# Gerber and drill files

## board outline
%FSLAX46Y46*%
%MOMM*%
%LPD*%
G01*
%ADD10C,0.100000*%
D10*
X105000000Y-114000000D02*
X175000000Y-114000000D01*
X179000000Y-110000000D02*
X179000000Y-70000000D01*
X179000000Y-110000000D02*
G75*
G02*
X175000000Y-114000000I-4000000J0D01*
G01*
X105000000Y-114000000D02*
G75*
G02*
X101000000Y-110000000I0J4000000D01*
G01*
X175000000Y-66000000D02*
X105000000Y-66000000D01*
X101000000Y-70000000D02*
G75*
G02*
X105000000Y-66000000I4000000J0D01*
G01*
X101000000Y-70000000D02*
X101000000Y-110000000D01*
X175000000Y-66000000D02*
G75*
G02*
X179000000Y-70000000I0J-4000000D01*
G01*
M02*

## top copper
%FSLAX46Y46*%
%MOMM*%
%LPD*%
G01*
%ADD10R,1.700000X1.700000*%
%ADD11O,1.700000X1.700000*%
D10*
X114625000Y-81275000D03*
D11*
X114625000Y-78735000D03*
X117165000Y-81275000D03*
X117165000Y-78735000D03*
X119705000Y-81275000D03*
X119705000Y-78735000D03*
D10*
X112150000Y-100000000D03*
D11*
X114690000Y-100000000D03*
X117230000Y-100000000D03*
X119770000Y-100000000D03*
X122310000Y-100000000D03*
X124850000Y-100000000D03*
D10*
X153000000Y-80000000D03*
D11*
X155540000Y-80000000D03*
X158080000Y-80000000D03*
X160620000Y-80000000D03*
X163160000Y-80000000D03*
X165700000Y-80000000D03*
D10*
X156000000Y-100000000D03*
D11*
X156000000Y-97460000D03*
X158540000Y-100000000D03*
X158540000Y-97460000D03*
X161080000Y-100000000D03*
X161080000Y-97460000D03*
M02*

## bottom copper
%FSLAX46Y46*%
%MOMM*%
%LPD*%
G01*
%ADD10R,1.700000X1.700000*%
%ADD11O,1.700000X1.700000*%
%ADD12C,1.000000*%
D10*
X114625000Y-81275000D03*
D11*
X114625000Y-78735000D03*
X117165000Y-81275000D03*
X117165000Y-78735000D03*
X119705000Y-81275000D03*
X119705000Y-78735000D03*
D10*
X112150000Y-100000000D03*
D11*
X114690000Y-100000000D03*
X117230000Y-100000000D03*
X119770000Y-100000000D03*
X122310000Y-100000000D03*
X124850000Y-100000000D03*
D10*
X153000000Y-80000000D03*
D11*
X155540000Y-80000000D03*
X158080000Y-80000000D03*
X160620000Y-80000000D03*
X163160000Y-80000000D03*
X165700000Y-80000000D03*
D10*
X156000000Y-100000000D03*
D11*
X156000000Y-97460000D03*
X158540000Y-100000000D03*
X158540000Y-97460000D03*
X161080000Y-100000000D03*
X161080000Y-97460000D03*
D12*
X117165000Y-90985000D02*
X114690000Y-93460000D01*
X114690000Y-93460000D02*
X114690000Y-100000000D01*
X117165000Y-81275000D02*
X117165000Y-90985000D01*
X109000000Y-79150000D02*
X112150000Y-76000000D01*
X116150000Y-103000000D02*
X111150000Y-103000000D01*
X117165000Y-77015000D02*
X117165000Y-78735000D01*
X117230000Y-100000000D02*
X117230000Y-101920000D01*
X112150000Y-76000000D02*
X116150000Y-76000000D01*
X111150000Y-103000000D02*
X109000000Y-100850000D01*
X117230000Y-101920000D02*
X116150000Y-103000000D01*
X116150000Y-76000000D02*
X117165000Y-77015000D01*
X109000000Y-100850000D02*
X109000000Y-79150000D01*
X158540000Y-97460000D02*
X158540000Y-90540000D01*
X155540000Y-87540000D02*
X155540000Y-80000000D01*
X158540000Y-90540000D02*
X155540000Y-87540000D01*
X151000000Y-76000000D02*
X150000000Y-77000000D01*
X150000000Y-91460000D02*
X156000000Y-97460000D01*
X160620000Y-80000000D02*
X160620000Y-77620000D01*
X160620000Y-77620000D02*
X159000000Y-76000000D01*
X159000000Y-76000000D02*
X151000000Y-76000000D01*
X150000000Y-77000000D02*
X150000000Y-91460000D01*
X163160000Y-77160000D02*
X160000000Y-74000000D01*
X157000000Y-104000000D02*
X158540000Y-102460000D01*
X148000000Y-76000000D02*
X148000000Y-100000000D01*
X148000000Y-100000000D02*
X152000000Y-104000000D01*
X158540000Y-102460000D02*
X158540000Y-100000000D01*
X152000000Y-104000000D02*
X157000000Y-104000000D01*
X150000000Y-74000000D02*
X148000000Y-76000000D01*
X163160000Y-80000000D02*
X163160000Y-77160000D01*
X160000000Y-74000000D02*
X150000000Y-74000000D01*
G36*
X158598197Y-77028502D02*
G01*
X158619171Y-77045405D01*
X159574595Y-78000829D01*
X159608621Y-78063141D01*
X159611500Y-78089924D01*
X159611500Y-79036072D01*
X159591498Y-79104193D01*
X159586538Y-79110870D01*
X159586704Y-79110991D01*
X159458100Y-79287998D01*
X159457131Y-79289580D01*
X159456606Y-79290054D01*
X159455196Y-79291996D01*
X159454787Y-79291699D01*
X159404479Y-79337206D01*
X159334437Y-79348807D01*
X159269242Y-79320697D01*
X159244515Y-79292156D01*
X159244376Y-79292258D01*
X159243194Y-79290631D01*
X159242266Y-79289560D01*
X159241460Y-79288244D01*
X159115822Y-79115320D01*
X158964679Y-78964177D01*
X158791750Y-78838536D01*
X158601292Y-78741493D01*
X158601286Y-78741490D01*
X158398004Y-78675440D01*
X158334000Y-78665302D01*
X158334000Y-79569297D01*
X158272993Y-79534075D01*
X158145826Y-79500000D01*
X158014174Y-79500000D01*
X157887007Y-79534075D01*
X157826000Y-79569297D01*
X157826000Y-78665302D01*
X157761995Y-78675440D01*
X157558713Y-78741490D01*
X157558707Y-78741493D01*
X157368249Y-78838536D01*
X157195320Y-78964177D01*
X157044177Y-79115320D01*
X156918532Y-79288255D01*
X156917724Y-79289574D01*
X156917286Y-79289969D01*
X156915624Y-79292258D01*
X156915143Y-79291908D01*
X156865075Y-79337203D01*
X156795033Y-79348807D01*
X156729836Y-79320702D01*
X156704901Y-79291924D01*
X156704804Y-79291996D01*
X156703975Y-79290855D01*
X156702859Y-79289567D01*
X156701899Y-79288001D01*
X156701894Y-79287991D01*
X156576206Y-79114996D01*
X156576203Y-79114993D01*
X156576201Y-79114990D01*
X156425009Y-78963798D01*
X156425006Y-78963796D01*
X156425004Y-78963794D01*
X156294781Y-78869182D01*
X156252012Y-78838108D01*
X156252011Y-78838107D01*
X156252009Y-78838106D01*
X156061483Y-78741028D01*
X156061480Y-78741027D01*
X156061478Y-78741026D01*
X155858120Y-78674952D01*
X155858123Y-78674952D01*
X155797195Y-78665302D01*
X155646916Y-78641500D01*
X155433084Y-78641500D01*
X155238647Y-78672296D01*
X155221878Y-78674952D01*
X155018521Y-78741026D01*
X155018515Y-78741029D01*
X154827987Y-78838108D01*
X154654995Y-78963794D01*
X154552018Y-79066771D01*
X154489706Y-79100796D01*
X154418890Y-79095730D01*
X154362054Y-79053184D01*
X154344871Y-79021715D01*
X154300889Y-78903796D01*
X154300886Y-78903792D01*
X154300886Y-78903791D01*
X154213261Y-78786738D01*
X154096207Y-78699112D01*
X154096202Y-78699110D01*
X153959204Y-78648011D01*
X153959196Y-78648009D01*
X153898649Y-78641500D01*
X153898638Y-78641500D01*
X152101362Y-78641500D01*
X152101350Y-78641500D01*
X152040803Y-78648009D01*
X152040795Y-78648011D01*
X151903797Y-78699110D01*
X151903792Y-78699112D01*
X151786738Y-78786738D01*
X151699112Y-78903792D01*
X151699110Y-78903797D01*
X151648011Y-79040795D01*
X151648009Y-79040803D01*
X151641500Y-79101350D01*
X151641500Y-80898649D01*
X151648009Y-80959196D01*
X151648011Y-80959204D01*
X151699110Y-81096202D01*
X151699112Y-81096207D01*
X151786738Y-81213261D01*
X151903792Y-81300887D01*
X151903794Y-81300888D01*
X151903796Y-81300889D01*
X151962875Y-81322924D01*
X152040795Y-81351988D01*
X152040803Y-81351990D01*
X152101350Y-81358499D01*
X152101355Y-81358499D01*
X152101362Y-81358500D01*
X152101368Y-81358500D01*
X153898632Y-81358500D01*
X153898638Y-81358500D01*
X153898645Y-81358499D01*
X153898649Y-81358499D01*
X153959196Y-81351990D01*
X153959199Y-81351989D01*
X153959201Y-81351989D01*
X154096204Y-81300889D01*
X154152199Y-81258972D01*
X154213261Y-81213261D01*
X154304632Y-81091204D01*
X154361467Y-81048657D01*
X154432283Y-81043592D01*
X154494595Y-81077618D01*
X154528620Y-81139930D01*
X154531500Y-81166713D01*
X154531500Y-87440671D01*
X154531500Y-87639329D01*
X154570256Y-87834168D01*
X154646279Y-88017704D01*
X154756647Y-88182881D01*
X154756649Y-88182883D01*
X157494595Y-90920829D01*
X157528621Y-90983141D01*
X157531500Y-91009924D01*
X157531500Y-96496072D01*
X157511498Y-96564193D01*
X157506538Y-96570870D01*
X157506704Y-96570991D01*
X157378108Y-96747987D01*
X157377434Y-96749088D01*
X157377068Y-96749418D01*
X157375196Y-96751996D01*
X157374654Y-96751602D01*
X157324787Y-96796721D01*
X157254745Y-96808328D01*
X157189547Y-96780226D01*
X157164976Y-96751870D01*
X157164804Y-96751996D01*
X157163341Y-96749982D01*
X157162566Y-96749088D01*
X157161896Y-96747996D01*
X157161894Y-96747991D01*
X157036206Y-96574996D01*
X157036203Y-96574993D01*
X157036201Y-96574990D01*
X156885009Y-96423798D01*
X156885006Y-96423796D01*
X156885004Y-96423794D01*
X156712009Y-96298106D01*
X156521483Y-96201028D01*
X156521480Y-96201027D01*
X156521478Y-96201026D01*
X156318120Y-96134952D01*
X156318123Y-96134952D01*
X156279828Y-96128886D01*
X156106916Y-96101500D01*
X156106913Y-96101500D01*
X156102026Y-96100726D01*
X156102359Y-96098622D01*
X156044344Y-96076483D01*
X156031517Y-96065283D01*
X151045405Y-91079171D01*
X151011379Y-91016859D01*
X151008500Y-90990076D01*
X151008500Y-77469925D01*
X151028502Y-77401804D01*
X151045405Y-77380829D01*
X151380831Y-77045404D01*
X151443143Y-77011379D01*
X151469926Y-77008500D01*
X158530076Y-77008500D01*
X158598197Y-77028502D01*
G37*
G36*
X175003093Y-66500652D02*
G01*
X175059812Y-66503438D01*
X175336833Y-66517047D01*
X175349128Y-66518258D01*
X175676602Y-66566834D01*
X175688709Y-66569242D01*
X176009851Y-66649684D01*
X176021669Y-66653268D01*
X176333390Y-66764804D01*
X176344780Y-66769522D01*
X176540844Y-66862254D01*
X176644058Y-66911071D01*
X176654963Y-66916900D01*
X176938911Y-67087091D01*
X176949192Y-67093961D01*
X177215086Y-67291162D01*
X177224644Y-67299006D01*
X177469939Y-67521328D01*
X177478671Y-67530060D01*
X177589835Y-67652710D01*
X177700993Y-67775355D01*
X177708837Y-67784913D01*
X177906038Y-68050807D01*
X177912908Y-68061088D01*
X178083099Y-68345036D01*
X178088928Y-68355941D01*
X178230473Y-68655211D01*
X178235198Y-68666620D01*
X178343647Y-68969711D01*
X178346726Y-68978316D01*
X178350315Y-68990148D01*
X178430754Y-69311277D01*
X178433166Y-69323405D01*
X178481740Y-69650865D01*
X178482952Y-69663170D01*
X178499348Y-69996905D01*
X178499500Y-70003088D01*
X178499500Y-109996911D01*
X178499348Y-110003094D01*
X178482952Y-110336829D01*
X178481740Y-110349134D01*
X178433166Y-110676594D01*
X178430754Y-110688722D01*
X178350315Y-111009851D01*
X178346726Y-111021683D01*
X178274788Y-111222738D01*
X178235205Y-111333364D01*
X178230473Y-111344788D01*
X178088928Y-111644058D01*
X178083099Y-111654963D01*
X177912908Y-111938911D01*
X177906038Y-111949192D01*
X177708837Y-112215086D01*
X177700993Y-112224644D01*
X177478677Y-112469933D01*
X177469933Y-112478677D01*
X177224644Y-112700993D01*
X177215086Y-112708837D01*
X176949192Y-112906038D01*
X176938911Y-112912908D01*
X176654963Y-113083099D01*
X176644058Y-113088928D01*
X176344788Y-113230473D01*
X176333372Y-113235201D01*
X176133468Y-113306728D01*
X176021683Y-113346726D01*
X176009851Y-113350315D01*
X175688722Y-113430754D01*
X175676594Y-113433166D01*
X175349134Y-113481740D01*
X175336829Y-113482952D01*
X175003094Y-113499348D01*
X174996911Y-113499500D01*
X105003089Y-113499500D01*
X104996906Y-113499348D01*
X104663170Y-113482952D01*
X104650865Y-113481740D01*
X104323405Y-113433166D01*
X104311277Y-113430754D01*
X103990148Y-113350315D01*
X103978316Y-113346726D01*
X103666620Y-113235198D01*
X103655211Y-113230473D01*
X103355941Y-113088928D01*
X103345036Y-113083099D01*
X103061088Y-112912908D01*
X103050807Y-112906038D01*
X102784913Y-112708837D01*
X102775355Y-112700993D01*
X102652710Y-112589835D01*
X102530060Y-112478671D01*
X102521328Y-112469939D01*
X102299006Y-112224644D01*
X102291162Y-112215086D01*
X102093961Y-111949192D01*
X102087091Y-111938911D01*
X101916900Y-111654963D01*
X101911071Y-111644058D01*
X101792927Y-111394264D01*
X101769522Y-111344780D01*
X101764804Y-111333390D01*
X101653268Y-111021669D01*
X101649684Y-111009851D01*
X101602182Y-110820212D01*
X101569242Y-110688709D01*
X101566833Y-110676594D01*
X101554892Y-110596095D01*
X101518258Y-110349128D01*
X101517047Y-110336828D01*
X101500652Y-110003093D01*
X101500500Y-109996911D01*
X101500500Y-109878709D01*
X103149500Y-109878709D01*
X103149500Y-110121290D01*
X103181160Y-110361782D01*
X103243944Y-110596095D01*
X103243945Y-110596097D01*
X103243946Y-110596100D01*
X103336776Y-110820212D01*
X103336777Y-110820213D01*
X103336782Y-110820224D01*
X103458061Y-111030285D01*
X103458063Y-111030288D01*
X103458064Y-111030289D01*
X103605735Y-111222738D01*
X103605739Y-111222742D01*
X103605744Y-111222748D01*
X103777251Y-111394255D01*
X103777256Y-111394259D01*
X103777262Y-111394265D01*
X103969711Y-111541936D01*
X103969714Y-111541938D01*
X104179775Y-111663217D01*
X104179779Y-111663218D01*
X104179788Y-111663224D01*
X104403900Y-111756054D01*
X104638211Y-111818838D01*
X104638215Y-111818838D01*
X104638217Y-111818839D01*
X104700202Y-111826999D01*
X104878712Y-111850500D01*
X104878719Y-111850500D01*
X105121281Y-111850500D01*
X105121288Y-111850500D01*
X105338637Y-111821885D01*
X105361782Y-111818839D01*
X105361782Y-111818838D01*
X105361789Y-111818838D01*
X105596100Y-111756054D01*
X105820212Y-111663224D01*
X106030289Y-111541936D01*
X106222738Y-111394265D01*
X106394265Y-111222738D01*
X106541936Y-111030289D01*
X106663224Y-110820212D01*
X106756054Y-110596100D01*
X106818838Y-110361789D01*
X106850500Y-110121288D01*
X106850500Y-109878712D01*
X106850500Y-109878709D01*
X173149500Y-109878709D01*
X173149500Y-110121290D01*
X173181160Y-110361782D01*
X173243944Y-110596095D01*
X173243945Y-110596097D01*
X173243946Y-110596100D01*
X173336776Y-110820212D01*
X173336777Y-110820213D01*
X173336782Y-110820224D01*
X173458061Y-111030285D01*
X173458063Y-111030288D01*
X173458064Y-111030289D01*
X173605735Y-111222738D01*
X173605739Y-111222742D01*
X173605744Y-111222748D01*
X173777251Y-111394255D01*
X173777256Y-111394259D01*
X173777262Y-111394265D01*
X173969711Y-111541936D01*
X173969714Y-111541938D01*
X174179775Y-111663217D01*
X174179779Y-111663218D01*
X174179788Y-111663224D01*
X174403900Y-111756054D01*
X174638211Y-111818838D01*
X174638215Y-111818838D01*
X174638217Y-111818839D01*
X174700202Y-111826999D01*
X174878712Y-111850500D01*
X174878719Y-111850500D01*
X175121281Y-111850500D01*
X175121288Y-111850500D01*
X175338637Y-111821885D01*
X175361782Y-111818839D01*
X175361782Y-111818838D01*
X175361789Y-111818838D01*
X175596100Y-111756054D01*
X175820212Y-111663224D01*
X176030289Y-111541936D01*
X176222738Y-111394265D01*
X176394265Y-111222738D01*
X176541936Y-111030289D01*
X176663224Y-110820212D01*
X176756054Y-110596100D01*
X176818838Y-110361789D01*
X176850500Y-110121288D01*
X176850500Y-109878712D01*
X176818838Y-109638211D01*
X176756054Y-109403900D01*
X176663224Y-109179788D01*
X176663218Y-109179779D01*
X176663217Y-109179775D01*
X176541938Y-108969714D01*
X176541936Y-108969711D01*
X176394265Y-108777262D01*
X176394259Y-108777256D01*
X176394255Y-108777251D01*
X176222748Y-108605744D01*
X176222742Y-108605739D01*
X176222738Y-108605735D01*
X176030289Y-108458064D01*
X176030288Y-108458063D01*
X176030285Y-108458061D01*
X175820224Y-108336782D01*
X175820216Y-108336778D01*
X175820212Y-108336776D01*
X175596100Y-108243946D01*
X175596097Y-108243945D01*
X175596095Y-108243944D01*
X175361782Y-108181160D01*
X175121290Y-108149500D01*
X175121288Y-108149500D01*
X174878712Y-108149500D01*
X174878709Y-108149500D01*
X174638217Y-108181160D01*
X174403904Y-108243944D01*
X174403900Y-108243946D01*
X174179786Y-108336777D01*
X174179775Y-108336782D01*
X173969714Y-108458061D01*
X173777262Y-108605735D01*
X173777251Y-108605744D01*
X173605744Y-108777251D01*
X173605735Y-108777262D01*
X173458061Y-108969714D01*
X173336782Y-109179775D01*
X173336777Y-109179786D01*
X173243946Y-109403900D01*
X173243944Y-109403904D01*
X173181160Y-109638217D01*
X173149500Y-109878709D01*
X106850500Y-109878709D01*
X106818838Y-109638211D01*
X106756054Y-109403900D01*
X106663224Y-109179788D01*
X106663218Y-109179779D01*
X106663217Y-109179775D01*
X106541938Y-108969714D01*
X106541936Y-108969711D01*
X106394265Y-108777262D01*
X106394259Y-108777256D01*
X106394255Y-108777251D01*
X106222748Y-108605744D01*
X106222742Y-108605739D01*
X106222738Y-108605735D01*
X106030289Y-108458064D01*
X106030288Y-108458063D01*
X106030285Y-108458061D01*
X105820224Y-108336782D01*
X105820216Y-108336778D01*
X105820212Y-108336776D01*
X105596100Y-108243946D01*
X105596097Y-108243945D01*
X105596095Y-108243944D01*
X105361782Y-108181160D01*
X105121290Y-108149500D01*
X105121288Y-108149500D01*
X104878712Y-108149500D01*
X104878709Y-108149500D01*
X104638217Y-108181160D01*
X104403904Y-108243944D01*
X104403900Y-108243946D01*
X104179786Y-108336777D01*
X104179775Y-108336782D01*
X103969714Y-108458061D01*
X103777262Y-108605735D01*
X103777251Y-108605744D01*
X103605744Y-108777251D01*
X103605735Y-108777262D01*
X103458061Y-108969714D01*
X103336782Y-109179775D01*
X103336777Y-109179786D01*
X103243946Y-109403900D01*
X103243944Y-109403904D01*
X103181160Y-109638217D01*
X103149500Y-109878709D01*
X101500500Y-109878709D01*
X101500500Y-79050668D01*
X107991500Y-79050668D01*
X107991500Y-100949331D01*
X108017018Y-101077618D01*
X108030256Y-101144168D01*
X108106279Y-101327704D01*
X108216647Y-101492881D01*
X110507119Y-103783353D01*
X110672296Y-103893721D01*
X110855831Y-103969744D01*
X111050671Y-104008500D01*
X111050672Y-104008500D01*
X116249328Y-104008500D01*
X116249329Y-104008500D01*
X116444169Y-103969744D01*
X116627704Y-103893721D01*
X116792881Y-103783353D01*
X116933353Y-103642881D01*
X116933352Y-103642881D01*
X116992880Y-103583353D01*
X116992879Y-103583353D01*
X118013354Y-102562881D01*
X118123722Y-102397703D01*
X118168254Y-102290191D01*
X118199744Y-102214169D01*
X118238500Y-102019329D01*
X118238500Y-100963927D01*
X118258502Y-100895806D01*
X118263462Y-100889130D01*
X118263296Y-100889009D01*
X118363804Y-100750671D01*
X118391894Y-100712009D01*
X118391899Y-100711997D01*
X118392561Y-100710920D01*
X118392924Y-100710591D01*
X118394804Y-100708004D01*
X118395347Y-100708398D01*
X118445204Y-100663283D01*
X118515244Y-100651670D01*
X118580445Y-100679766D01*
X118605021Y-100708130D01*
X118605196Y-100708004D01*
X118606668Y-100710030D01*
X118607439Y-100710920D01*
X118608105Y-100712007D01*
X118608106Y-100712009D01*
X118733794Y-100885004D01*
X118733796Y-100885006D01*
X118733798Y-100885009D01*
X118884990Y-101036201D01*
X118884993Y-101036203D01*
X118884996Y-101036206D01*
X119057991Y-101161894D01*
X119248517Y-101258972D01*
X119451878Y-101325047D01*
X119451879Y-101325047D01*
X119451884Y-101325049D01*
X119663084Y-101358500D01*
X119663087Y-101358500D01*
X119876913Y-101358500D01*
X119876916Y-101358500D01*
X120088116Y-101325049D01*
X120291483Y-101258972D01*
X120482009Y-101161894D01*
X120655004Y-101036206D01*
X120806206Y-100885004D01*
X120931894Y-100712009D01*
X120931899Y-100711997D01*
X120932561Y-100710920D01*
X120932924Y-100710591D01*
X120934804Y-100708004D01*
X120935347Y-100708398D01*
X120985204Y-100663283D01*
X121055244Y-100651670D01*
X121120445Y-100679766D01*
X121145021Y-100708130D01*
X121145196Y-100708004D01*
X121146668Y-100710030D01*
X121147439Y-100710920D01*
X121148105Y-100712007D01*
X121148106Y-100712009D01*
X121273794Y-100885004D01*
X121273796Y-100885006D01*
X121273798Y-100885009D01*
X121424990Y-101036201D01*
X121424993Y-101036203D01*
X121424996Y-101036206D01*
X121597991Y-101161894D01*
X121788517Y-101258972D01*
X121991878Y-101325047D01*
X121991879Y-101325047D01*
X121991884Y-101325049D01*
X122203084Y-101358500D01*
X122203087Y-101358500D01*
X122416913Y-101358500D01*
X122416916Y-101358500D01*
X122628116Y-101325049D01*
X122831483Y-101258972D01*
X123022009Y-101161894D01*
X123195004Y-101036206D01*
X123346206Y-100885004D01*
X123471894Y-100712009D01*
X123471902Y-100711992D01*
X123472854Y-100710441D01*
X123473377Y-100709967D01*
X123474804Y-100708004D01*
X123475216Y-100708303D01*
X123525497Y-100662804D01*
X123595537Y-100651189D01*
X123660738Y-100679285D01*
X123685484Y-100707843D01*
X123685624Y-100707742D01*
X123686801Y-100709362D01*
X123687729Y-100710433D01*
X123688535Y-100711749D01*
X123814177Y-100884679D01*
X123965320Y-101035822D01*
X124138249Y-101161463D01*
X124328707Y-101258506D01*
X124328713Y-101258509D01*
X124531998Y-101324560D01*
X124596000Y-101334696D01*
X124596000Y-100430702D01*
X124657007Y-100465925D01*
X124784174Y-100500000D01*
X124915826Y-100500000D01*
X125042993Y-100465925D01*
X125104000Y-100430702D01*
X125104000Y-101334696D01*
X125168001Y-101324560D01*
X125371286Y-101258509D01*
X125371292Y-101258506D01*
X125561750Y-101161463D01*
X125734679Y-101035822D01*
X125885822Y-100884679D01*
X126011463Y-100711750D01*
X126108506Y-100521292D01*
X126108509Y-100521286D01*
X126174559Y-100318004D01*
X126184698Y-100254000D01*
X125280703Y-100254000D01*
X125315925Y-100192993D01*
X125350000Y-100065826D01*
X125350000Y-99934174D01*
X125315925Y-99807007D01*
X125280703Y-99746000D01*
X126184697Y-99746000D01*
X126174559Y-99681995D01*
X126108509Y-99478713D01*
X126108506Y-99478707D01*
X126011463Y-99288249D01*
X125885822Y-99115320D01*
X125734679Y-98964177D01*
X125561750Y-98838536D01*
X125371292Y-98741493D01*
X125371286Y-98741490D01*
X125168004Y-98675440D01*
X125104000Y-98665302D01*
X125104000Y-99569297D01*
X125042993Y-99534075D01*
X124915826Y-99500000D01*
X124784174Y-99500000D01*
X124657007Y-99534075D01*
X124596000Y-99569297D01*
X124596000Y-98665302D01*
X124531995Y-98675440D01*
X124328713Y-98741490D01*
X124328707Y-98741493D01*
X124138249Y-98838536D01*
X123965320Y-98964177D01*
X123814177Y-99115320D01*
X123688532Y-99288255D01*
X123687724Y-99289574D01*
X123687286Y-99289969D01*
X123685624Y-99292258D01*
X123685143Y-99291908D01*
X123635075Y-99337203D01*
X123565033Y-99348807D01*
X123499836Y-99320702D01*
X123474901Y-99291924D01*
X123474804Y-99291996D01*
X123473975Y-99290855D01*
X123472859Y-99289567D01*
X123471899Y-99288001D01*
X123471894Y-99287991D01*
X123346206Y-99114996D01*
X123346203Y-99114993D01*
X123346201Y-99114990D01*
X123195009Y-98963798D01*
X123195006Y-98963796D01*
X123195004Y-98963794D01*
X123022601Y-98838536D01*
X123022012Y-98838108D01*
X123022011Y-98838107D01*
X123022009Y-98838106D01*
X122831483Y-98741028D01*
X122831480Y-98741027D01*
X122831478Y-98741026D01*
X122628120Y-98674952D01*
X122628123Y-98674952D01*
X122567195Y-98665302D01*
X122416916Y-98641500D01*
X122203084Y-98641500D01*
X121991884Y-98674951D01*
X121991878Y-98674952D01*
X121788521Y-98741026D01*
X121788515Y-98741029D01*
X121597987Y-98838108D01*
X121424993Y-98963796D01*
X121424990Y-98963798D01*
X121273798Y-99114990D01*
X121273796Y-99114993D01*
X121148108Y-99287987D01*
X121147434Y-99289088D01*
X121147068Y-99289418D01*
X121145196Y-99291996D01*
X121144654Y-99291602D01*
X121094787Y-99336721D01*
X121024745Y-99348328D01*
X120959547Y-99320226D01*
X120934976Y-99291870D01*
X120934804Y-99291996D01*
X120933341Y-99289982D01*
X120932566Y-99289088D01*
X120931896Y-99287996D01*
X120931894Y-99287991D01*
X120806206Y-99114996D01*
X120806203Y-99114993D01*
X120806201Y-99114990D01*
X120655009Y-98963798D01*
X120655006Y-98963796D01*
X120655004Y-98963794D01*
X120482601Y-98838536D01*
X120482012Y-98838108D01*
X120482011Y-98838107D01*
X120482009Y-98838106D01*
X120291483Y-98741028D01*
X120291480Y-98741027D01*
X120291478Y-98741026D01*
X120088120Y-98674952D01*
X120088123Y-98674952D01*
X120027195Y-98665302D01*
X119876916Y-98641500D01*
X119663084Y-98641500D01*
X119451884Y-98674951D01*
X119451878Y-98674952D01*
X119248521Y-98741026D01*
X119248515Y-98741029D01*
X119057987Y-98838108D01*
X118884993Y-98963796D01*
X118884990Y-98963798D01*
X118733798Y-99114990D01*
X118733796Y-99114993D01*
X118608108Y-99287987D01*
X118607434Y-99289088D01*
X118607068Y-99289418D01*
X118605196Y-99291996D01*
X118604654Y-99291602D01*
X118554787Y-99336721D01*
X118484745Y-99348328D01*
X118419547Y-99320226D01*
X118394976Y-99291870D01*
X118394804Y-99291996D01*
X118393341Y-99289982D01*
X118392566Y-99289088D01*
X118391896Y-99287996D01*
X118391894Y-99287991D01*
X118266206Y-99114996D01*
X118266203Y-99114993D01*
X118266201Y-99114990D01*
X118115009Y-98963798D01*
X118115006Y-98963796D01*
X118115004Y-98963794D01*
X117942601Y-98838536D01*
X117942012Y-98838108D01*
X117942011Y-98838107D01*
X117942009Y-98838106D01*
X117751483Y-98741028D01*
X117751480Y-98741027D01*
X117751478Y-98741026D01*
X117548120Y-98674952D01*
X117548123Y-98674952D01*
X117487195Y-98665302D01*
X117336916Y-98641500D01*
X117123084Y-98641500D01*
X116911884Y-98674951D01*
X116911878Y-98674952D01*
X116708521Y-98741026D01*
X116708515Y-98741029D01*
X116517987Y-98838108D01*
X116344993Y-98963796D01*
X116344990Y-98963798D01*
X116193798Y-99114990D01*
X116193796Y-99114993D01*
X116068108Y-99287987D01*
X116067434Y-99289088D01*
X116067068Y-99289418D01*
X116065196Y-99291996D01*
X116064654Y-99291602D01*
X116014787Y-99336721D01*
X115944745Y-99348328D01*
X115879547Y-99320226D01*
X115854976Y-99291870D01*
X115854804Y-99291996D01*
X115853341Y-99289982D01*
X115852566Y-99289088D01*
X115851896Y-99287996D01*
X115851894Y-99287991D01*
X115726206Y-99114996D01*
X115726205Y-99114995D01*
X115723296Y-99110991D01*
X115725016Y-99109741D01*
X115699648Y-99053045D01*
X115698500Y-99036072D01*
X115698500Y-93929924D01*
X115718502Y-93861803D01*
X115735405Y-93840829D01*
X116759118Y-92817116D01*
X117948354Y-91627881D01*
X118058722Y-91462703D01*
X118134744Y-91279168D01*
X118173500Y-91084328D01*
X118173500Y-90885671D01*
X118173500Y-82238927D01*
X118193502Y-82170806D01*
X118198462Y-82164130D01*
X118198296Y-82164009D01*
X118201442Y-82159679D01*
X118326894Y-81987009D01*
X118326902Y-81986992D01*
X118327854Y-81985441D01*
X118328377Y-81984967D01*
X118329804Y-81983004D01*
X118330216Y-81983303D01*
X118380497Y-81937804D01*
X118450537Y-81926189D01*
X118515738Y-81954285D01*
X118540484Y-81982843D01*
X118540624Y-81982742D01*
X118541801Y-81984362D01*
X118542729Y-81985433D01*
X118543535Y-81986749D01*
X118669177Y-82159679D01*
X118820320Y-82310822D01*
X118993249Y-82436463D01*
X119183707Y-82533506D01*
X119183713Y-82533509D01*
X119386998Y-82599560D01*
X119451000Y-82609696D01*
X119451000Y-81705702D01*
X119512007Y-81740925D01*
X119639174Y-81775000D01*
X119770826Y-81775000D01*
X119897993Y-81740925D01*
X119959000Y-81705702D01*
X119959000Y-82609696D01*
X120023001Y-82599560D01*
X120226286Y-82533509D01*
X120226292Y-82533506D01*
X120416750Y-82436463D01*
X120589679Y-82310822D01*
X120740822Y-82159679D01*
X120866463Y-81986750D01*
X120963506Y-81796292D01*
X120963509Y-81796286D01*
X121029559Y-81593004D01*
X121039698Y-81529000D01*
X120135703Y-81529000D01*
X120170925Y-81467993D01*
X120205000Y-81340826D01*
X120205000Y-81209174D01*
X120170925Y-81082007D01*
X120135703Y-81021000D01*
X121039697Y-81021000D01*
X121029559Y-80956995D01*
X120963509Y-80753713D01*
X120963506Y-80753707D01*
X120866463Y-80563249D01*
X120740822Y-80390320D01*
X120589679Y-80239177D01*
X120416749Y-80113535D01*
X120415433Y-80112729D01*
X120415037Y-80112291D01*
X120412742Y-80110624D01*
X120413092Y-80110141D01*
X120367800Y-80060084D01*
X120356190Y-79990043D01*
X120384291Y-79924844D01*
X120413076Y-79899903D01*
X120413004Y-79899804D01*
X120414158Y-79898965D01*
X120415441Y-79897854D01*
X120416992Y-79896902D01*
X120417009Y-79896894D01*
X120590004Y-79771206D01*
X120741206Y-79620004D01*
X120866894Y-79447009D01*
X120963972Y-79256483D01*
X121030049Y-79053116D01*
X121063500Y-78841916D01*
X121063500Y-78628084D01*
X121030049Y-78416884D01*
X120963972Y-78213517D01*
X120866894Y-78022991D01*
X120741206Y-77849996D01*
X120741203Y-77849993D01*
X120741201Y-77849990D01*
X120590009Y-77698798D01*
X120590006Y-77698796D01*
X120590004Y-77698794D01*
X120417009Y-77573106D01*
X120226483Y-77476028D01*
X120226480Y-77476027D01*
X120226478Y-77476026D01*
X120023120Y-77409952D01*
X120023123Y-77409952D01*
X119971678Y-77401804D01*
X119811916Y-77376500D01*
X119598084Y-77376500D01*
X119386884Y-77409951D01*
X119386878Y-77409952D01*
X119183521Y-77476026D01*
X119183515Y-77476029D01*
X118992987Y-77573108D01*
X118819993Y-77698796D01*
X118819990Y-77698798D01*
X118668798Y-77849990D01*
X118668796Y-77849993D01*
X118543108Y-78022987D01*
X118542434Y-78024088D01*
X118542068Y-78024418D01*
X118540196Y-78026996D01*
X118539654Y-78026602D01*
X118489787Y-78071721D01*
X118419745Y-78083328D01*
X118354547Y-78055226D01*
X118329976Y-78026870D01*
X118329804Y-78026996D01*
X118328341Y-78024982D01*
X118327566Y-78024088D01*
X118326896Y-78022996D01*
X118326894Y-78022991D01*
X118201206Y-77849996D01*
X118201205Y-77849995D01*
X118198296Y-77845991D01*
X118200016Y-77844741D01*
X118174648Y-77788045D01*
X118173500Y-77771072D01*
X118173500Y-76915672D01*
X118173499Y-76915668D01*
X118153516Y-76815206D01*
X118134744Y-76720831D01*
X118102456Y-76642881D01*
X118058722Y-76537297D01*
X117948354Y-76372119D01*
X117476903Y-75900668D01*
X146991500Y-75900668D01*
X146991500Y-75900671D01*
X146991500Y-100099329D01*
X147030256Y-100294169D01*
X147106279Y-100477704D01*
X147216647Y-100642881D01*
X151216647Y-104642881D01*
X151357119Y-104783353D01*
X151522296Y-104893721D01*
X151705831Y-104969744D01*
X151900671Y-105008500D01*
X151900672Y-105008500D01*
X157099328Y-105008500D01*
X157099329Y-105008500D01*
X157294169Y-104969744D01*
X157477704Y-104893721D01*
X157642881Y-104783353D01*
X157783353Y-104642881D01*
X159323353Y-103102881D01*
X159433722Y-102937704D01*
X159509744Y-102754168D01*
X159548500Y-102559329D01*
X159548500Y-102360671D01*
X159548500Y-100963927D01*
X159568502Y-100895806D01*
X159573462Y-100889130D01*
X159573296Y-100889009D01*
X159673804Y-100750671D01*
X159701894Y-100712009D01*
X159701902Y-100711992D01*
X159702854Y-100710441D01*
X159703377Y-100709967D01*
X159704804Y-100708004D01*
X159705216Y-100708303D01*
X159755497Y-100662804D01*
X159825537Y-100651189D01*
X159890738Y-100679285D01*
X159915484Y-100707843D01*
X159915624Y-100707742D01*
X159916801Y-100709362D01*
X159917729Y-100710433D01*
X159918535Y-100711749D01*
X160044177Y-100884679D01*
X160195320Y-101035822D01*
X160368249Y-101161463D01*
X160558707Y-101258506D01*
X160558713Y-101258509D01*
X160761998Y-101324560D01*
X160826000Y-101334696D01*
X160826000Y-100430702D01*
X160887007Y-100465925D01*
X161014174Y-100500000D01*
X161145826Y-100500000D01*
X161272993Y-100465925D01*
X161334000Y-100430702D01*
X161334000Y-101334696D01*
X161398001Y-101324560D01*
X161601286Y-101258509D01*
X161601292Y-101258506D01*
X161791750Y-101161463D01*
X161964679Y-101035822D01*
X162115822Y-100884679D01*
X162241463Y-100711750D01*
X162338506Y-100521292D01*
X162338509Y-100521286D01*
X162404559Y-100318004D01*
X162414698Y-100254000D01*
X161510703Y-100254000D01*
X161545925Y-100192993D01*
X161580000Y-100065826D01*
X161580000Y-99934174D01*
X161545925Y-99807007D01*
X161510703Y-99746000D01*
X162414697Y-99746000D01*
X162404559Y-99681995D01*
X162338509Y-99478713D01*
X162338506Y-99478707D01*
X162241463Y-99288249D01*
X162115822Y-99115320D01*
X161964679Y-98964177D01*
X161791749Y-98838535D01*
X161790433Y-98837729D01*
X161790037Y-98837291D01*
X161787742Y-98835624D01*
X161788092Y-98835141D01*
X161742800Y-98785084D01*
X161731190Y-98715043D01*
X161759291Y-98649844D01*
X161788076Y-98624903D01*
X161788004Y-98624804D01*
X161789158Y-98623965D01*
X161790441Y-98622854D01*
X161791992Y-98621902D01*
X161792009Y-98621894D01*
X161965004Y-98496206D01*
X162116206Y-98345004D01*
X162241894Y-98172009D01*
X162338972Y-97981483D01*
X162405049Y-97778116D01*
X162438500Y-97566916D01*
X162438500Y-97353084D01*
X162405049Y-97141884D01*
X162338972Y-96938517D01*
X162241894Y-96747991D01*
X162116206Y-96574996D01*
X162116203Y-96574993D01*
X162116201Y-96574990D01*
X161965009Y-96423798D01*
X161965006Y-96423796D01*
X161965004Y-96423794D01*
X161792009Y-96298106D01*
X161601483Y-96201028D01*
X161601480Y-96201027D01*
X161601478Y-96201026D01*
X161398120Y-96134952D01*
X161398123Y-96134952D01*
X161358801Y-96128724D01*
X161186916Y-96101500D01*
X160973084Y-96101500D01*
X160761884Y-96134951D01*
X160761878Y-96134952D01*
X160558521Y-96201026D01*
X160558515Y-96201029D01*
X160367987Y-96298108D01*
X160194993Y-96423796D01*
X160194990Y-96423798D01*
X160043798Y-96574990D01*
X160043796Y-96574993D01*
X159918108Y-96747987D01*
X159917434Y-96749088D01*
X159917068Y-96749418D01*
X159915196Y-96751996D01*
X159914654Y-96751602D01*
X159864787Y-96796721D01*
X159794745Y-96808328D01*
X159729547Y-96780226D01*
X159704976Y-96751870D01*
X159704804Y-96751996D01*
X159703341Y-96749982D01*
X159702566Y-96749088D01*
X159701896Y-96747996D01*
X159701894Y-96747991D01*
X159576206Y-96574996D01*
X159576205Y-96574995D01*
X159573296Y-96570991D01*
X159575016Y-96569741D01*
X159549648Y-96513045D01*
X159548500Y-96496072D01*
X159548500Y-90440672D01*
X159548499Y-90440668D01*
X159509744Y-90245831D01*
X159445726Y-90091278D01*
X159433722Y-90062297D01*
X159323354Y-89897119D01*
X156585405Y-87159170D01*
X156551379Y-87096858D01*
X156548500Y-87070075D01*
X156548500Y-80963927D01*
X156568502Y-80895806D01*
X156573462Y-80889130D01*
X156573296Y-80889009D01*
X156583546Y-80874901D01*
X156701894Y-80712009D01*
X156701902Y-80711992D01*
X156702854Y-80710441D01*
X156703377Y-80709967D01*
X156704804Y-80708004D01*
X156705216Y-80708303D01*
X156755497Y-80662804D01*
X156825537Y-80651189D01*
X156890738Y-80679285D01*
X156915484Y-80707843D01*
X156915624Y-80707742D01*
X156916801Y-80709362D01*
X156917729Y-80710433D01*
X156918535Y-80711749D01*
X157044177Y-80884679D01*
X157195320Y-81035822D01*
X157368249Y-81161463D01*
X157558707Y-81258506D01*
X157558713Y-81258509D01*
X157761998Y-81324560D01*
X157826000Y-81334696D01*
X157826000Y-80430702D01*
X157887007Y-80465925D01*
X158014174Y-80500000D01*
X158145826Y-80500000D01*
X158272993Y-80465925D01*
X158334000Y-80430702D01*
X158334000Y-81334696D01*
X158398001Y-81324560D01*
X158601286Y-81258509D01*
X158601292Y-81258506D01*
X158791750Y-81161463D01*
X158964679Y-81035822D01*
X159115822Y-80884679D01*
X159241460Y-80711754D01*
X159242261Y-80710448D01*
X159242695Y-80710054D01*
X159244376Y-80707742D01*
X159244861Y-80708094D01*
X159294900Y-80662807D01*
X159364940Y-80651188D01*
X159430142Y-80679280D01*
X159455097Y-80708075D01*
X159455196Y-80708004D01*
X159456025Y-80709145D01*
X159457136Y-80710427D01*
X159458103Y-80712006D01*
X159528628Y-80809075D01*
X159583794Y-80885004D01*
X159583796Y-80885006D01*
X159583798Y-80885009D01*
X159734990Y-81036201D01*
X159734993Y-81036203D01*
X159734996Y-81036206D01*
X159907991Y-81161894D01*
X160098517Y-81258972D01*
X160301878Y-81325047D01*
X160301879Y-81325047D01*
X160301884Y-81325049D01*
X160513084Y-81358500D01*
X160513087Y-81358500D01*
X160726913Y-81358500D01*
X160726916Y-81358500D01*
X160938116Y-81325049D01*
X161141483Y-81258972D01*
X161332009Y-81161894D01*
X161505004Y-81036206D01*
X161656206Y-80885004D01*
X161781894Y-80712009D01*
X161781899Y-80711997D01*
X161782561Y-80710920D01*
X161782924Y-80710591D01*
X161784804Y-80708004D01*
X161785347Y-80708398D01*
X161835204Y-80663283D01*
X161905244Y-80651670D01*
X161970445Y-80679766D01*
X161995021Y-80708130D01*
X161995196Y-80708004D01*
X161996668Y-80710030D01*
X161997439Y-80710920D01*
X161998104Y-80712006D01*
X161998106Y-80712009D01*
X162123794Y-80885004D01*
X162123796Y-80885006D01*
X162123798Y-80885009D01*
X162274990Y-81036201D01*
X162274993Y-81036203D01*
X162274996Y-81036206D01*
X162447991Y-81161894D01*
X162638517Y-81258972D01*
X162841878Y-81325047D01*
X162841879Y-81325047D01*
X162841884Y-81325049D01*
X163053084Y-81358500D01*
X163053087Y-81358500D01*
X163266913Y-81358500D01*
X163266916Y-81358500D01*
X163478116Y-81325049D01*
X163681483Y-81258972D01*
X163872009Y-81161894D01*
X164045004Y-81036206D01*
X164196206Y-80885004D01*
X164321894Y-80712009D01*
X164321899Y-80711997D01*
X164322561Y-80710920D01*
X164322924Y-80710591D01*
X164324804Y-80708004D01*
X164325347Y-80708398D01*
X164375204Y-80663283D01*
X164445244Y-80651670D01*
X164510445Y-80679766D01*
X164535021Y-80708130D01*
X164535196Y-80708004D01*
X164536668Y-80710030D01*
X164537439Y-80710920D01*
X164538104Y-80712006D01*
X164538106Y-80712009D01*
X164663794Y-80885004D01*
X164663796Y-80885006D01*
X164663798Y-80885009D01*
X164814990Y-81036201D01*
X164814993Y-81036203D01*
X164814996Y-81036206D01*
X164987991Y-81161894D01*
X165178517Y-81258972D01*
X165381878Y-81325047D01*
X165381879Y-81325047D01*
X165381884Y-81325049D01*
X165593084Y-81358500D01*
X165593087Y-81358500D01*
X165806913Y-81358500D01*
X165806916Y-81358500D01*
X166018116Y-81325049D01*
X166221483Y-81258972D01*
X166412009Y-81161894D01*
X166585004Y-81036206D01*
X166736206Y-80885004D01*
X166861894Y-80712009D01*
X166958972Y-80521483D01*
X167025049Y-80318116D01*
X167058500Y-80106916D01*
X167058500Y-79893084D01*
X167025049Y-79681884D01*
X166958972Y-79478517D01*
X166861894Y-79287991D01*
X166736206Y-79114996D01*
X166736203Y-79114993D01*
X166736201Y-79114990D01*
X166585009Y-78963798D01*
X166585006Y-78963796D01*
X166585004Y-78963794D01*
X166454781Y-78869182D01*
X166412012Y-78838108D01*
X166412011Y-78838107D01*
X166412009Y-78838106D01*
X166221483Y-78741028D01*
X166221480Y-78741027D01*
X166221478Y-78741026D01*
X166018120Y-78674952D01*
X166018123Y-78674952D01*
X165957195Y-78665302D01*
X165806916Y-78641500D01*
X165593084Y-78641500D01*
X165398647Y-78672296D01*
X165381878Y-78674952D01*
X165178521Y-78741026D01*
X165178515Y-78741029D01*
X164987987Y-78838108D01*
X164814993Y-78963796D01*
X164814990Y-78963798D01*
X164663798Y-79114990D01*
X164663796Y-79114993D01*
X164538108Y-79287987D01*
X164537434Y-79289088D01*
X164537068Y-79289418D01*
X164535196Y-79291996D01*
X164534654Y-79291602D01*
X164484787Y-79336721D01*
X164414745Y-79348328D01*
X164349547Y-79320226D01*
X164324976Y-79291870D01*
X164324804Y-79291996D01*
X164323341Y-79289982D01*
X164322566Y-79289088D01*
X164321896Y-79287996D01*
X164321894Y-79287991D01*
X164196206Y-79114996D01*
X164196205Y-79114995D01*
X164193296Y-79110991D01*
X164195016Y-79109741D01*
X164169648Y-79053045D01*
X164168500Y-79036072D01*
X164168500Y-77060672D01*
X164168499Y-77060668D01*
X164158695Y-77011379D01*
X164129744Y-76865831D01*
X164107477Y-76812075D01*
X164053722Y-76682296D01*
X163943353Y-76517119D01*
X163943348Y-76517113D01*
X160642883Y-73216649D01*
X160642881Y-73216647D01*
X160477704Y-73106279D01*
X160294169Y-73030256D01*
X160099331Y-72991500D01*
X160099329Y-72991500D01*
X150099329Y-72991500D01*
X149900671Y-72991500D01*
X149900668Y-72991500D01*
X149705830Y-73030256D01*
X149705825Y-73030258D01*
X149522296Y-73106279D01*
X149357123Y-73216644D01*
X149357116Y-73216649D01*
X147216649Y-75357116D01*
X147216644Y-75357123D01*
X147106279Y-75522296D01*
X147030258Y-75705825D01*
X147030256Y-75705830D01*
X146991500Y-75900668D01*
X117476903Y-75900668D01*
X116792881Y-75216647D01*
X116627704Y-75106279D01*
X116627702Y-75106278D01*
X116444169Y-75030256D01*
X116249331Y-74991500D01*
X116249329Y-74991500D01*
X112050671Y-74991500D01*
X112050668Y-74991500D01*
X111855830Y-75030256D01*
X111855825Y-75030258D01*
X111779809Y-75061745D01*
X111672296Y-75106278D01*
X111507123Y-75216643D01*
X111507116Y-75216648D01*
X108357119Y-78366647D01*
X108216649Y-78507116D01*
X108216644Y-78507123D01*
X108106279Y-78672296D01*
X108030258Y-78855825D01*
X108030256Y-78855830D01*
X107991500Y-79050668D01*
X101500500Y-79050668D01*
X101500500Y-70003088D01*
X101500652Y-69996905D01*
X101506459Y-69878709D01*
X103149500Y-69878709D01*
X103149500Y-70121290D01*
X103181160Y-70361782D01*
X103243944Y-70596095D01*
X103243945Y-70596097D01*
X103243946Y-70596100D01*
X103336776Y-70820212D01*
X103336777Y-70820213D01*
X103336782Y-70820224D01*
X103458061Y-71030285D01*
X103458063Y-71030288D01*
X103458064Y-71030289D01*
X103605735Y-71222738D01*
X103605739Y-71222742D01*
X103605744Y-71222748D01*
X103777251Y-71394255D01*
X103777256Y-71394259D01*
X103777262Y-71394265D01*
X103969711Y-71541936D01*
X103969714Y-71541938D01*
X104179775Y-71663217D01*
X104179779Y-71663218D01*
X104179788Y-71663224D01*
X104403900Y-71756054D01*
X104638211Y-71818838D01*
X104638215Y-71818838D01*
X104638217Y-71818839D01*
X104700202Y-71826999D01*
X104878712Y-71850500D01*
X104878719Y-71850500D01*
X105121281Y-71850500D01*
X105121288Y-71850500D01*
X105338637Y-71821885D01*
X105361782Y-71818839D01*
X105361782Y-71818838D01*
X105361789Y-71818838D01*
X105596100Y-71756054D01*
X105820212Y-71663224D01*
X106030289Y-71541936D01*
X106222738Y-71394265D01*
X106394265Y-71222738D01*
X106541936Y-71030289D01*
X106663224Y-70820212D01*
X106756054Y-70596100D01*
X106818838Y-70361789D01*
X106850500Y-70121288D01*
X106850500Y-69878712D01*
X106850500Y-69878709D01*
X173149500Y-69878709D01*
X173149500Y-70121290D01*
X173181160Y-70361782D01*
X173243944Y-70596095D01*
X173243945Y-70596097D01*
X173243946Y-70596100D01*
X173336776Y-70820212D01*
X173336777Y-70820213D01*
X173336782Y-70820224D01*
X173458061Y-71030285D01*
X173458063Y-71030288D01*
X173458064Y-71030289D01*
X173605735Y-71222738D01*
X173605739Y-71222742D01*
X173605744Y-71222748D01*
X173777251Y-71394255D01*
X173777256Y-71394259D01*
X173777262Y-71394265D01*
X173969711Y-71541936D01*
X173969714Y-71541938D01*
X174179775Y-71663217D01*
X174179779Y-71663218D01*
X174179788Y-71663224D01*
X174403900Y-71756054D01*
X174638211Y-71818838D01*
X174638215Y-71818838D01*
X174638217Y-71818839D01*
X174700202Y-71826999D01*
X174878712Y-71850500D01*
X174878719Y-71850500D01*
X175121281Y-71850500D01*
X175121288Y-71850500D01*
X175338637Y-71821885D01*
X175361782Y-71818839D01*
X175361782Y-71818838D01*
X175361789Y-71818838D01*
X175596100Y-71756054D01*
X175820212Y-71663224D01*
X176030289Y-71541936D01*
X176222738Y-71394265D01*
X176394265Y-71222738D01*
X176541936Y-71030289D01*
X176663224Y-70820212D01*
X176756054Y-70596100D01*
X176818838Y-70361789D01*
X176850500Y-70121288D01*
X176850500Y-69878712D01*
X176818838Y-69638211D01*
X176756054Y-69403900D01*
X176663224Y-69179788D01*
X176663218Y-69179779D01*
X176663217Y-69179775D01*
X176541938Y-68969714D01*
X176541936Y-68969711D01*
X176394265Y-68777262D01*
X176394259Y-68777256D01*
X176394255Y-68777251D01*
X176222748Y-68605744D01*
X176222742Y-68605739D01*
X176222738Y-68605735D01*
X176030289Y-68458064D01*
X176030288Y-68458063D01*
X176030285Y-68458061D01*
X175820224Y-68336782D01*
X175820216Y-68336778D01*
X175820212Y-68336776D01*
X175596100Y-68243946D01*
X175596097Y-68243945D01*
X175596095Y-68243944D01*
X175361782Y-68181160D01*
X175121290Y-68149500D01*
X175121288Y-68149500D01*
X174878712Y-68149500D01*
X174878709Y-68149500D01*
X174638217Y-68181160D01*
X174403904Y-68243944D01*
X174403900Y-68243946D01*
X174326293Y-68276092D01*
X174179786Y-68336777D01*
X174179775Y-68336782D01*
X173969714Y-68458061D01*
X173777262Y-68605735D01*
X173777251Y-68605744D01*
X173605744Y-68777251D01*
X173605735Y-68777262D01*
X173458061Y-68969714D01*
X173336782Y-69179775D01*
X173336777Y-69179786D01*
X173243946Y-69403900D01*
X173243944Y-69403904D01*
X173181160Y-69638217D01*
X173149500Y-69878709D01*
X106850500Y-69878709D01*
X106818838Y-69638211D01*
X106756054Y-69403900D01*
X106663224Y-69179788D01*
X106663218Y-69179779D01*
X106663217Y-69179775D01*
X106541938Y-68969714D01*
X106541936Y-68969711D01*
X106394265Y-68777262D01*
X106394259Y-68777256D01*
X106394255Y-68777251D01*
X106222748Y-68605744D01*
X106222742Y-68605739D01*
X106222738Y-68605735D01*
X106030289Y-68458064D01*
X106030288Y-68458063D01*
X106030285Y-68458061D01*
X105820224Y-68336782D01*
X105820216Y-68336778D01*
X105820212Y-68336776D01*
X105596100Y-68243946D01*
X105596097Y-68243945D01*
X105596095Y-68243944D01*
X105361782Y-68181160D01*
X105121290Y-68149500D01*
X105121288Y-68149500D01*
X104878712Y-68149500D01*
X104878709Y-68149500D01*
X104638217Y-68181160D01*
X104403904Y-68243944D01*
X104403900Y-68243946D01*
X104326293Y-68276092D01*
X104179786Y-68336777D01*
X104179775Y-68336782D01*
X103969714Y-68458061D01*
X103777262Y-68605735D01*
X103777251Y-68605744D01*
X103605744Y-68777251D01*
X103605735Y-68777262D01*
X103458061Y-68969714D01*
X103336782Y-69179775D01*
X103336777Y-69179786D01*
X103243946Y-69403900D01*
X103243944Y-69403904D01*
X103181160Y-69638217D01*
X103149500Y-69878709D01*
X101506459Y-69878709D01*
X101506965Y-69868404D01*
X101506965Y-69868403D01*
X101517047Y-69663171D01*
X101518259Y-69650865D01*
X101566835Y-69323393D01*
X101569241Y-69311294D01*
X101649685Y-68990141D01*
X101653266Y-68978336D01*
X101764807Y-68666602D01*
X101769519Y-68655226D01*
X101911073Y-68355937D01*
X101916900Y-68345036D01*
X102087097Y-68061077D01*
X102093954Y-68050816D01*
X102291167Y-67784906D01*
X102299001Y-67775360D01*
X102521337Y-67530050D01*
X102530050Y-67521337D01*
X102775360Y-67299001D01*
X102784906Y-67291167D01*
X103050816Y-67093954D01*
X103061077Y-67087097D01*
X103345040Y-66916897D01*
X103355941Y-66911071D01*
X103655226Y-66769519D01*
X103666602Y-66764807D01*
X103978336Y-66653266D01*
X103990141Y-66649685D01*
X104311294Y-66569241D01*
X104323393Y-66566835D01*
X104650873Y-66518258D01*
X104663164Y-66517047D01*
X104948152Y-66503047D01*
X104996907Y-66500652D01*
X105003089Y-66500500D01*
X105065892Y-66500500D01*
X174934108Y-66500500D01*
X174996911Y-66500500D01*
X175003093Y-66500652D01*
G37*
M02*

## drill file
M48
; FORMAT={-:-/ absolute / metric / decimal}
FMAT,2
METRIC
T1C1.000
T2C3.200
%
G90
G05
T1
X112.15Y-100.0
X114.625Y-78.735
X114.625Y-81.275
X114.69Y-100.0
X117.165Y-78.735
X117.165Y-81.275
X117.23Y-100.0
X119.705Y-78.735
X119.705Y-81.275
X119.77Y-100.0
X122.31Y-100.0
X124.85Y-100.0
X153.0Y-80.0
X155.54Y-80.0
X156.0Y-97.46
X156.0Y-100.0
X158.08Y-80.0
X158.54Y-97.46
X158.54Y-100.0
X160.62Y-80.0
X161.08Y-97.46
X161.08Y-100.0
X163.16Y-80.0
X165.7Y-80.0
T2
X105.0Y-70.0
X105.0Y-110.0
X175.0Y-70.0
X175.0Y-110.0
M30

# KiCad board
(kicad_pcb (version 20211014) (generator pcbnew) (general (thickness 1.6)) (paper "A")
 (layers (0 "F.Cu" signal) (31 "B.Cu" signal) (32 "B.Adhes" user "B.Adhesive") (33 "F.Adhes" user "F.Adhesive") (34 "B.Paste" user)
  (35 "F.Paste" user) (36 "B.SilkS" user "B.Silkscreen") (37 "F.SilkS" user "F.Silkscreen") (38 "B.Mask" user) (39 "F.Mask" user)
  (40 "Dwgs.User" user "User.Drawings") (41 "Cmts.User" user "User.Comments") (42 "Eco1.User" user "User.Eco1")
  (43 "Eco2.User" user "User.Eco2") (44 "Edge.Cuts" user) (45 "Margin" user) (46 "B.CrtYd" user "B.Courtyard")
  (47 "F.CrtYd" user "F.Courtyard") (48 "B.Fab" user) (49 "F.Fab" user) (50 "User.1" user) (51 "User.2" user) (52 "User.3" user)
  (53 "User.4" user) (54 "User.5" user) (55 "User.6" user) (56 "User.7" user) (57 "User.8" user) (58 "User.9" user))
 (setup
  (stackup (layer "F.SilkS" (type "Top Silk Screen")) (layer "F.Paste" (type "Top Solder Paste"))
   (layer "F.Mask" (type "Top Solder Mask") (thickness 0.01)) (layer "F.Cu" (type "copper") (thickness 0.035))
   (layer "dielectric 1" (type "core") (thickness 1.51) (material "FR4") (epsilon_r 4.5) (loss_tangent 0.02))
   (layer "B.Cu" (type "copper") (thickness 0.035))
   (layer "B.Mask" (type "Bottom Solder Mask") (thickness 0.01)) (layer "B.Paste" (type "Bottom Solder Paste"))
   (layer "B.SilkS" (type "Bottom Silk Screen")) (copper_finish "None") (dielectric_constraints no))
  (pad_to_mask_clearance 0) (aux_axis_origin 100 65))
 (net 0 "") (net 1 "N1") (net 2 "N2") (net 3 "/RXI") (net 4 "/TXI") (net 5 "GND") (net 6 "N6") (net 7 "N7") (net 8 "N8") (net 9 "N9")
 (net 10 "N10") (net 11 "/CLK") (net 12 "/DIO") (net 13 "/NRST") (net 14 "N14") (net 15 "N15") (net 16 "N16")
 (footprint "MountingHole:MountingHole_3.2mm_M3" (layer "F.Cu") (at 105 70 90)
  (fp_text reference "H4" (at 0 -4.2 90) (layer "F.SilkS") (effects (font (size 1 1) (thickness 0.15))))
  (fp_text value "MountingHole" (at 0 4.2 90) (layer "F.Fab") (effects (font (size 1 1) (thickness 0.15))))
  (pad "" np_thru_hole circle (at 0 0 90) (size 3.2 3.2) (drill 3.2) (layers *.Cu *.Mask)))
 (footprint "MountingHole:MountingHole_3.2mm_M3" (layer "F.Cu") (at 175 70 90)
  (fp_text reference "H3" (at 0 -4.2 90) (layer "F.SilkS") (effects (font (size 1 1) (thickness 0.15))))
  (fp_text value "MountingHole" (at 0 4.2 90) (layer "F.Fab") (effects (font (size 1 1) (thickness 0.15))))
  (pad "" np_thru_hole circle (at 0 0 90) (size 3.2 3.2) (drill 3.2) (layers *.Cu *.Mask)))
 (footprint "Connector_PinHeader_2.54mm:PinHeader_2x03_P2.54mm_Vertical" (layer "F.Cu") (at 114.625 81.275 90)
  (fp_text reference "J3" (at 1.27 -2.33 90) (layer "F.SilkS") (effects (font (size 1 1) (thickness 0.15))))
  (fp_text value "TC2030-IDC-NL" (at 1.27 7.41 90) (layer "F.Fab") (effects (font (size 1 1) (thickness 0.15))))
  (pad "1" thru_hole rect (at 0 0 90) (size 1.7 1.7) (drill 1) (layers *.Cu *.Mask) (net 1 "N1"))
  (pad "2" thru_hole oval (at 2.54 0 90) (size 1.7 1.7) (drill 1) (layers *.Cu *.Mask) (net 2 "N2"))
  (pad "3" thru_hole oval (at 0 2.54 90) (size 1.7 1.7) (drill 1) (layers *.Cu *.Mask) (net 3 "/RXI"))
  (pad "4" thru_hole oval (at 2.54 2.54 90) (size 1.7 1.7) (drill 1) (layers *.Cu *.Mask) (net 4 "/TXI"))
  (pad "5" thru_hole oval (at 0 5.08 90) (size 1.7 1.7) (drill 1) (layers *.Cu *.Mask) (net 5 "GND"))
  (pad "6" thru_hole oval (at 2.54 5.08 90) (size 1.7 1.7) (drill 1) (layers *.Cu *.Mask) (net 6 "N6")))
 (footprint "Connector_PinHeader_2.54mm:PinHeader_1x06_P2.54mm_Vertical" (layer "F.Cu") (at 112.15 100 90)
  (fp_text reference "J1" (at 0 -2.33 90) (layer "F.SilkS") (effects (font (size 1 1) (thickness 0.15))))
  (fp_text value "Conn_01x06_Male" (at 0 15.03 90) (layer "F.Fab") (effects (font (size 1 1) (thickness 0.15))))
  (pad "1" thru_hole rect (at 0 0 90) (size 1.7 1.7) (drill 1) (layers *.Cu *.Mask) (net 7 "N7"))
  (pad "2" thru_hole oval (at 0 2.54 90) (size 1.7 1.7) (drill 1) (layers *.Cu *.Mask) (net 3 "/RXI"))
  (pad "3" thru_hole oval (at 0 5.08 90) (size 1.7 1.7) (drill 1) (layers *.Cu *.Mask) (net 4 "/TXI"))
  (pad "4" thru_hole oval (at 0 7.62 90) (size 1.7 1.7) (drill 1) (layers *.Cu *.Mask) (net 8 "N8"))
  (pad "5" thru_hole oval (at 0 10.16 90) (size 1.7 1.7) (drill 1) (layers *.Cu *.Mask) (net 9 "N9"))
  (pad "6" thru_hole oval (at 0 12.7 90) (size 1.7 1.7) (drill 1) (layers *.Cu *.Mask) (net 5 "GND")))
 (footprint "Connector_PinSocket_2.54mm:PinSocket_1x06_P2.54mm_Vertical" (layer "F.Cu") (at 153 80 90)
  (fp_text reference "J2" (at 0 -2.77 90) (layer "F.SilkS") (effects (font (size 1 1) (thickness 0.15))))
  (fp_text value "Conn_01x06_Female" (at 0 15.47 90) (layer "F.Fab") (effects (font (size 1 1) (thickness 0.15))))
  (pad "1" thru_hole rect (at 0 0 90) (size 1.7 1.7) (drill 1) (layers *.Cu *.Mask) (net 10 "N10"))
  (pad "2" thru_hole oval (at 0 2.54 90) (size 1.7 1.7) (drill 1) (layers *.Cu *.Mask) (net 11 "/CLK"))
  (pad "3" thru_hole oval (at 0 5.08 90) (size 1.7 1.7) (drill 1) (layers *.Cu *.Mask) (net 5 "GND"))
  (pad "4" thru_hole oval (at 0 7.62 90) (size 1.7 1.7) (drill 1) (layers *.Cu *.Mask) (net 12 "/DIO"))
  (pad "5" thru_hole oval (at 0 10.16 90) (size 1.7 1.7) (drill 1) (layers *.Cu *.Mask) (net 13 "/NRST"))
  (pad "6" thru_hole oval (at 0 12.7 90) (size 1.7 1.7) (drill 1) (layers *.Cu *.Mask) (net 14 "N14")))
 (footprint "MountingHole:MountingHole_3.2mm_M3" (layer "F.Cu") (at 175 110 90)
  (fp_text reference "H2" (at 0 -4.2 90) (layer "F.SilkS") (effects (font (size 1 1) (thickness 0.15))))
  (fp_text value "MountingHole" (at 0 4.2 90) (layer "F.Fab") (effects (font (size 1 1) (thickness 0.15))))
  (pad "" np_thru_hole circle (at 0 0 90) (size 3.2 3.2) (drill 3.2) (layers *.Cu *.Mask)))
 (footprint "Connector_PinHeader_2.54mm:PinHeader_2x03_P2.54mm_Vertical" (layer "F.Cu") (at 156 100 90)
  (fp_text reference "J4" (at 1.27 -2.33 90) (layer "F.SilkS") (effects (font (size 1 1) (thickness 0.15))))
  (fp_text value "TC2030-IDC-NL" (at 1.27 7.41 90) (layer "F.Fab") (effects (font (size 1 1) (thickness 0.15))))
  (pad "1" thru_hole rect (at 0 0 90) (size 1.7 1.7) (drill 1) (layers *.Cu *.Mask) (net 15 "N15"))
  (pad "2" thru_hole oval (at 2.54 0 90) (size 1.7 1.7) (drill 1) (layers *.Cu *.Mask) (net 12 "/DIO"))
  (pad "3" thru_hole oval (at 0 2.54 90) (size 1.7 1.7) (drill 1) (layers *.Cu *.Mask) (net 13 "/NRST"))
  (pad "4" thru_hole oval (at 2.54 2.54 90) (size 1.7 1.7) (drill 1) (layers *.Cu *.Mask) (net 11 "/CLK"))
  (pad "5" thru_hole oval (at 0 5.08 90) (size 1.7 1.7) (drill 1) (layers *.Cu *.Mask) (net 5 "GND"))
  (pad "6" thru_hole oval (at 2.54 5.08 90) (size 1.7 1.7) (drill 1) (layers *.Cu *.Mask) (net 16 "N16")))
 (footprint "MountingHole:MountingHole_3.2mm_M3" (layer "F.Cu") (at 105 110 90)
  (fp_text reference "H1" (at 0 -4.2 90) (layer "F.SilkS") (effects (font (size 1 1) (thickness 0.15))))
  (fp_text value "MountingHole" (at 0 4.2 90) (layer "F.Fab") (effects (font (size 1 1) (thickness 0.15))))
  (pad "" np_thru_hole circle (at 0 0 90) (size 3.2 3.2) (drill 3.2) (layers *.Cu *.Mask)))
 (gr_line (start 105 114) (end 175 114) (layer "Edge.Cuts") (width 0.1))
 (gr_line (start 179 110) (end 179 70) (layer "Edge.Cuts") (width 0.1))
 (gr_arc (start 179 110) (mid 177.828427 112.828427) (end 175 114) (layer "Edge.Cuts") (width 0.1))
 (gr_arc (start 105 114) (mid 102.171573 112.828427) (end 101 110) (layer "Edge.Cuts") (width 0.1))
 (gr_line (start 175 66) (end 105 66) (layer "Edge.Cuts") (width 0.1))
 (gr_arc (start 101 70) (mid 102.171573 67.171573) (end 105 66) (layer "Edge.Cuts") (width 0.1))
 (gr_line (start 101 70) (end 101 110) (layer "Edge.Cuts") (width 0.1))
 (gr_arc (start 175 66) (mid 177.828427 67.171573) (end 179 70) (layer "Edge.Cuts") (width 0.1))
 (segment (start 117.165 90.985) (end 114.69 93.46) (width 1) (layer "B.Cu") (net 3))
 (segment (start 114.69 93.46) (end 114.69 100) (width 1) (layer "B.Cu") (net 3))
 (segment (start 117.165 81.275) (end 117.165 90.985) (width 1) (layer "B.Cu") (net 3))
 (segment (start 109 79.15) (end 112.15 76) (width 1) (layer "B.Cu") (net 4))
 (segment (start 116.15 103) (end 111.15 103) (width 1) (layer "B.Cu") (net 4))
 (segment (start 117.165 77.015) (end 117.165 78.735) (width 1) (layer "B.Cu") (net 4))
 (segment (start 117.23 100) (end 117.23 101.92) (width 1) (layer "B.Cu") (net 4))
 (segment (start 112.15 76) (end 116.15 76) (width 1) (layer "B.Cu") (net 4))
 (segment (start 111.15 103) (end 109 100.85) (width 1) (layer "B.Cu") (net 4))
 (segment (start 117.23 101.92) (end 116.15 103) (width 1) (layer "B.Cu") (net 4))
 (segment (start 116.15 76) (end 117.165 77.015) (width 1) (layer "B.Cu") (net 4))
 (segment (start 109 100.85) (end 109 79.15) (width 1) (layer "B.Cu") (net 4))
 (segment (start 158.54 97.46) (end 158.54 90.54) (width 1) (layer "B.Cu") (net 11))
 (segment (start 155.54 87.54) (end 155.54 80) (width 1) (layer "B.Cu") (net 11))
 (segment (start 158.54 90.54) (end 155.54 87.54) (width 1) (layer "B.Cu") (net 11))
 (segment (start 151 76) (end 150 77) (width 1) (layer "B.Cu") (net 12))
 (segment (start 150 91.46) (end 156 97.46) (width 1) (layer "B.Cu") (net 12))
 (segment (start 160.62 80) (end 160.62 77.62) (width 1) (layer "B.Cu") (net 12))
 (segment (start 160.62 77.62) (end 159 76) (width 1) (layer "B.Cu") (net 12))
 (segment (start 159 76) (end 151 76) (width 1) (layer "B.Cu") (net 12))
 (segment (start 150 77) (end 150 91.46) (width 1) (layer "B.Cu") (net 12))
 (segment (start 163.16 77.16) (end 160 74) (width 1) (layer "B.Cu") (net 13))
 (segment (start 157 104) (end 158.54 102.46) (width 1) (layer "B.Cu") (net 13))
 (segment (start 148 76) (end 148 100) (width 1) (layer "B.Cu") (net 13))
 (segment (start 148 100) (end 152 104) (width 1) (layer "B.Cu") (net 13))
 (segment (start 158.54 102.46) (end 158.54 100) (width 1) (layer "B.Cu") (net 13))
 (segment (start 152 104) (end 157 104) (width 1) (layer "B.Cu") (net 13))
 (segment (start 150 74) (end 148 76) (width 1) (layer "B.Cu") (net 13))
 (segment (start 163.16 80) (end 163.16 77.16) (width 1) (layer "B.Cu") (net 13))
 (segment (start 160 74) (end 150 74) (width 1) (layer "B.Cu") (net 13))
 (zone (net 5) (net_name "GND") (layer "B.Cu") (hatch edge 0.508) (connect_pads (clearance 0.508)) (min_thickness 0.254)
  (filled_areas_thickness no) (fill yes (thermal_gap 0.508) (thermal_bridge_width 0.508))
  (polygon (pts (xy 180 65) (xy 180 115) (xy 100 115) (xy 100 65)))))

